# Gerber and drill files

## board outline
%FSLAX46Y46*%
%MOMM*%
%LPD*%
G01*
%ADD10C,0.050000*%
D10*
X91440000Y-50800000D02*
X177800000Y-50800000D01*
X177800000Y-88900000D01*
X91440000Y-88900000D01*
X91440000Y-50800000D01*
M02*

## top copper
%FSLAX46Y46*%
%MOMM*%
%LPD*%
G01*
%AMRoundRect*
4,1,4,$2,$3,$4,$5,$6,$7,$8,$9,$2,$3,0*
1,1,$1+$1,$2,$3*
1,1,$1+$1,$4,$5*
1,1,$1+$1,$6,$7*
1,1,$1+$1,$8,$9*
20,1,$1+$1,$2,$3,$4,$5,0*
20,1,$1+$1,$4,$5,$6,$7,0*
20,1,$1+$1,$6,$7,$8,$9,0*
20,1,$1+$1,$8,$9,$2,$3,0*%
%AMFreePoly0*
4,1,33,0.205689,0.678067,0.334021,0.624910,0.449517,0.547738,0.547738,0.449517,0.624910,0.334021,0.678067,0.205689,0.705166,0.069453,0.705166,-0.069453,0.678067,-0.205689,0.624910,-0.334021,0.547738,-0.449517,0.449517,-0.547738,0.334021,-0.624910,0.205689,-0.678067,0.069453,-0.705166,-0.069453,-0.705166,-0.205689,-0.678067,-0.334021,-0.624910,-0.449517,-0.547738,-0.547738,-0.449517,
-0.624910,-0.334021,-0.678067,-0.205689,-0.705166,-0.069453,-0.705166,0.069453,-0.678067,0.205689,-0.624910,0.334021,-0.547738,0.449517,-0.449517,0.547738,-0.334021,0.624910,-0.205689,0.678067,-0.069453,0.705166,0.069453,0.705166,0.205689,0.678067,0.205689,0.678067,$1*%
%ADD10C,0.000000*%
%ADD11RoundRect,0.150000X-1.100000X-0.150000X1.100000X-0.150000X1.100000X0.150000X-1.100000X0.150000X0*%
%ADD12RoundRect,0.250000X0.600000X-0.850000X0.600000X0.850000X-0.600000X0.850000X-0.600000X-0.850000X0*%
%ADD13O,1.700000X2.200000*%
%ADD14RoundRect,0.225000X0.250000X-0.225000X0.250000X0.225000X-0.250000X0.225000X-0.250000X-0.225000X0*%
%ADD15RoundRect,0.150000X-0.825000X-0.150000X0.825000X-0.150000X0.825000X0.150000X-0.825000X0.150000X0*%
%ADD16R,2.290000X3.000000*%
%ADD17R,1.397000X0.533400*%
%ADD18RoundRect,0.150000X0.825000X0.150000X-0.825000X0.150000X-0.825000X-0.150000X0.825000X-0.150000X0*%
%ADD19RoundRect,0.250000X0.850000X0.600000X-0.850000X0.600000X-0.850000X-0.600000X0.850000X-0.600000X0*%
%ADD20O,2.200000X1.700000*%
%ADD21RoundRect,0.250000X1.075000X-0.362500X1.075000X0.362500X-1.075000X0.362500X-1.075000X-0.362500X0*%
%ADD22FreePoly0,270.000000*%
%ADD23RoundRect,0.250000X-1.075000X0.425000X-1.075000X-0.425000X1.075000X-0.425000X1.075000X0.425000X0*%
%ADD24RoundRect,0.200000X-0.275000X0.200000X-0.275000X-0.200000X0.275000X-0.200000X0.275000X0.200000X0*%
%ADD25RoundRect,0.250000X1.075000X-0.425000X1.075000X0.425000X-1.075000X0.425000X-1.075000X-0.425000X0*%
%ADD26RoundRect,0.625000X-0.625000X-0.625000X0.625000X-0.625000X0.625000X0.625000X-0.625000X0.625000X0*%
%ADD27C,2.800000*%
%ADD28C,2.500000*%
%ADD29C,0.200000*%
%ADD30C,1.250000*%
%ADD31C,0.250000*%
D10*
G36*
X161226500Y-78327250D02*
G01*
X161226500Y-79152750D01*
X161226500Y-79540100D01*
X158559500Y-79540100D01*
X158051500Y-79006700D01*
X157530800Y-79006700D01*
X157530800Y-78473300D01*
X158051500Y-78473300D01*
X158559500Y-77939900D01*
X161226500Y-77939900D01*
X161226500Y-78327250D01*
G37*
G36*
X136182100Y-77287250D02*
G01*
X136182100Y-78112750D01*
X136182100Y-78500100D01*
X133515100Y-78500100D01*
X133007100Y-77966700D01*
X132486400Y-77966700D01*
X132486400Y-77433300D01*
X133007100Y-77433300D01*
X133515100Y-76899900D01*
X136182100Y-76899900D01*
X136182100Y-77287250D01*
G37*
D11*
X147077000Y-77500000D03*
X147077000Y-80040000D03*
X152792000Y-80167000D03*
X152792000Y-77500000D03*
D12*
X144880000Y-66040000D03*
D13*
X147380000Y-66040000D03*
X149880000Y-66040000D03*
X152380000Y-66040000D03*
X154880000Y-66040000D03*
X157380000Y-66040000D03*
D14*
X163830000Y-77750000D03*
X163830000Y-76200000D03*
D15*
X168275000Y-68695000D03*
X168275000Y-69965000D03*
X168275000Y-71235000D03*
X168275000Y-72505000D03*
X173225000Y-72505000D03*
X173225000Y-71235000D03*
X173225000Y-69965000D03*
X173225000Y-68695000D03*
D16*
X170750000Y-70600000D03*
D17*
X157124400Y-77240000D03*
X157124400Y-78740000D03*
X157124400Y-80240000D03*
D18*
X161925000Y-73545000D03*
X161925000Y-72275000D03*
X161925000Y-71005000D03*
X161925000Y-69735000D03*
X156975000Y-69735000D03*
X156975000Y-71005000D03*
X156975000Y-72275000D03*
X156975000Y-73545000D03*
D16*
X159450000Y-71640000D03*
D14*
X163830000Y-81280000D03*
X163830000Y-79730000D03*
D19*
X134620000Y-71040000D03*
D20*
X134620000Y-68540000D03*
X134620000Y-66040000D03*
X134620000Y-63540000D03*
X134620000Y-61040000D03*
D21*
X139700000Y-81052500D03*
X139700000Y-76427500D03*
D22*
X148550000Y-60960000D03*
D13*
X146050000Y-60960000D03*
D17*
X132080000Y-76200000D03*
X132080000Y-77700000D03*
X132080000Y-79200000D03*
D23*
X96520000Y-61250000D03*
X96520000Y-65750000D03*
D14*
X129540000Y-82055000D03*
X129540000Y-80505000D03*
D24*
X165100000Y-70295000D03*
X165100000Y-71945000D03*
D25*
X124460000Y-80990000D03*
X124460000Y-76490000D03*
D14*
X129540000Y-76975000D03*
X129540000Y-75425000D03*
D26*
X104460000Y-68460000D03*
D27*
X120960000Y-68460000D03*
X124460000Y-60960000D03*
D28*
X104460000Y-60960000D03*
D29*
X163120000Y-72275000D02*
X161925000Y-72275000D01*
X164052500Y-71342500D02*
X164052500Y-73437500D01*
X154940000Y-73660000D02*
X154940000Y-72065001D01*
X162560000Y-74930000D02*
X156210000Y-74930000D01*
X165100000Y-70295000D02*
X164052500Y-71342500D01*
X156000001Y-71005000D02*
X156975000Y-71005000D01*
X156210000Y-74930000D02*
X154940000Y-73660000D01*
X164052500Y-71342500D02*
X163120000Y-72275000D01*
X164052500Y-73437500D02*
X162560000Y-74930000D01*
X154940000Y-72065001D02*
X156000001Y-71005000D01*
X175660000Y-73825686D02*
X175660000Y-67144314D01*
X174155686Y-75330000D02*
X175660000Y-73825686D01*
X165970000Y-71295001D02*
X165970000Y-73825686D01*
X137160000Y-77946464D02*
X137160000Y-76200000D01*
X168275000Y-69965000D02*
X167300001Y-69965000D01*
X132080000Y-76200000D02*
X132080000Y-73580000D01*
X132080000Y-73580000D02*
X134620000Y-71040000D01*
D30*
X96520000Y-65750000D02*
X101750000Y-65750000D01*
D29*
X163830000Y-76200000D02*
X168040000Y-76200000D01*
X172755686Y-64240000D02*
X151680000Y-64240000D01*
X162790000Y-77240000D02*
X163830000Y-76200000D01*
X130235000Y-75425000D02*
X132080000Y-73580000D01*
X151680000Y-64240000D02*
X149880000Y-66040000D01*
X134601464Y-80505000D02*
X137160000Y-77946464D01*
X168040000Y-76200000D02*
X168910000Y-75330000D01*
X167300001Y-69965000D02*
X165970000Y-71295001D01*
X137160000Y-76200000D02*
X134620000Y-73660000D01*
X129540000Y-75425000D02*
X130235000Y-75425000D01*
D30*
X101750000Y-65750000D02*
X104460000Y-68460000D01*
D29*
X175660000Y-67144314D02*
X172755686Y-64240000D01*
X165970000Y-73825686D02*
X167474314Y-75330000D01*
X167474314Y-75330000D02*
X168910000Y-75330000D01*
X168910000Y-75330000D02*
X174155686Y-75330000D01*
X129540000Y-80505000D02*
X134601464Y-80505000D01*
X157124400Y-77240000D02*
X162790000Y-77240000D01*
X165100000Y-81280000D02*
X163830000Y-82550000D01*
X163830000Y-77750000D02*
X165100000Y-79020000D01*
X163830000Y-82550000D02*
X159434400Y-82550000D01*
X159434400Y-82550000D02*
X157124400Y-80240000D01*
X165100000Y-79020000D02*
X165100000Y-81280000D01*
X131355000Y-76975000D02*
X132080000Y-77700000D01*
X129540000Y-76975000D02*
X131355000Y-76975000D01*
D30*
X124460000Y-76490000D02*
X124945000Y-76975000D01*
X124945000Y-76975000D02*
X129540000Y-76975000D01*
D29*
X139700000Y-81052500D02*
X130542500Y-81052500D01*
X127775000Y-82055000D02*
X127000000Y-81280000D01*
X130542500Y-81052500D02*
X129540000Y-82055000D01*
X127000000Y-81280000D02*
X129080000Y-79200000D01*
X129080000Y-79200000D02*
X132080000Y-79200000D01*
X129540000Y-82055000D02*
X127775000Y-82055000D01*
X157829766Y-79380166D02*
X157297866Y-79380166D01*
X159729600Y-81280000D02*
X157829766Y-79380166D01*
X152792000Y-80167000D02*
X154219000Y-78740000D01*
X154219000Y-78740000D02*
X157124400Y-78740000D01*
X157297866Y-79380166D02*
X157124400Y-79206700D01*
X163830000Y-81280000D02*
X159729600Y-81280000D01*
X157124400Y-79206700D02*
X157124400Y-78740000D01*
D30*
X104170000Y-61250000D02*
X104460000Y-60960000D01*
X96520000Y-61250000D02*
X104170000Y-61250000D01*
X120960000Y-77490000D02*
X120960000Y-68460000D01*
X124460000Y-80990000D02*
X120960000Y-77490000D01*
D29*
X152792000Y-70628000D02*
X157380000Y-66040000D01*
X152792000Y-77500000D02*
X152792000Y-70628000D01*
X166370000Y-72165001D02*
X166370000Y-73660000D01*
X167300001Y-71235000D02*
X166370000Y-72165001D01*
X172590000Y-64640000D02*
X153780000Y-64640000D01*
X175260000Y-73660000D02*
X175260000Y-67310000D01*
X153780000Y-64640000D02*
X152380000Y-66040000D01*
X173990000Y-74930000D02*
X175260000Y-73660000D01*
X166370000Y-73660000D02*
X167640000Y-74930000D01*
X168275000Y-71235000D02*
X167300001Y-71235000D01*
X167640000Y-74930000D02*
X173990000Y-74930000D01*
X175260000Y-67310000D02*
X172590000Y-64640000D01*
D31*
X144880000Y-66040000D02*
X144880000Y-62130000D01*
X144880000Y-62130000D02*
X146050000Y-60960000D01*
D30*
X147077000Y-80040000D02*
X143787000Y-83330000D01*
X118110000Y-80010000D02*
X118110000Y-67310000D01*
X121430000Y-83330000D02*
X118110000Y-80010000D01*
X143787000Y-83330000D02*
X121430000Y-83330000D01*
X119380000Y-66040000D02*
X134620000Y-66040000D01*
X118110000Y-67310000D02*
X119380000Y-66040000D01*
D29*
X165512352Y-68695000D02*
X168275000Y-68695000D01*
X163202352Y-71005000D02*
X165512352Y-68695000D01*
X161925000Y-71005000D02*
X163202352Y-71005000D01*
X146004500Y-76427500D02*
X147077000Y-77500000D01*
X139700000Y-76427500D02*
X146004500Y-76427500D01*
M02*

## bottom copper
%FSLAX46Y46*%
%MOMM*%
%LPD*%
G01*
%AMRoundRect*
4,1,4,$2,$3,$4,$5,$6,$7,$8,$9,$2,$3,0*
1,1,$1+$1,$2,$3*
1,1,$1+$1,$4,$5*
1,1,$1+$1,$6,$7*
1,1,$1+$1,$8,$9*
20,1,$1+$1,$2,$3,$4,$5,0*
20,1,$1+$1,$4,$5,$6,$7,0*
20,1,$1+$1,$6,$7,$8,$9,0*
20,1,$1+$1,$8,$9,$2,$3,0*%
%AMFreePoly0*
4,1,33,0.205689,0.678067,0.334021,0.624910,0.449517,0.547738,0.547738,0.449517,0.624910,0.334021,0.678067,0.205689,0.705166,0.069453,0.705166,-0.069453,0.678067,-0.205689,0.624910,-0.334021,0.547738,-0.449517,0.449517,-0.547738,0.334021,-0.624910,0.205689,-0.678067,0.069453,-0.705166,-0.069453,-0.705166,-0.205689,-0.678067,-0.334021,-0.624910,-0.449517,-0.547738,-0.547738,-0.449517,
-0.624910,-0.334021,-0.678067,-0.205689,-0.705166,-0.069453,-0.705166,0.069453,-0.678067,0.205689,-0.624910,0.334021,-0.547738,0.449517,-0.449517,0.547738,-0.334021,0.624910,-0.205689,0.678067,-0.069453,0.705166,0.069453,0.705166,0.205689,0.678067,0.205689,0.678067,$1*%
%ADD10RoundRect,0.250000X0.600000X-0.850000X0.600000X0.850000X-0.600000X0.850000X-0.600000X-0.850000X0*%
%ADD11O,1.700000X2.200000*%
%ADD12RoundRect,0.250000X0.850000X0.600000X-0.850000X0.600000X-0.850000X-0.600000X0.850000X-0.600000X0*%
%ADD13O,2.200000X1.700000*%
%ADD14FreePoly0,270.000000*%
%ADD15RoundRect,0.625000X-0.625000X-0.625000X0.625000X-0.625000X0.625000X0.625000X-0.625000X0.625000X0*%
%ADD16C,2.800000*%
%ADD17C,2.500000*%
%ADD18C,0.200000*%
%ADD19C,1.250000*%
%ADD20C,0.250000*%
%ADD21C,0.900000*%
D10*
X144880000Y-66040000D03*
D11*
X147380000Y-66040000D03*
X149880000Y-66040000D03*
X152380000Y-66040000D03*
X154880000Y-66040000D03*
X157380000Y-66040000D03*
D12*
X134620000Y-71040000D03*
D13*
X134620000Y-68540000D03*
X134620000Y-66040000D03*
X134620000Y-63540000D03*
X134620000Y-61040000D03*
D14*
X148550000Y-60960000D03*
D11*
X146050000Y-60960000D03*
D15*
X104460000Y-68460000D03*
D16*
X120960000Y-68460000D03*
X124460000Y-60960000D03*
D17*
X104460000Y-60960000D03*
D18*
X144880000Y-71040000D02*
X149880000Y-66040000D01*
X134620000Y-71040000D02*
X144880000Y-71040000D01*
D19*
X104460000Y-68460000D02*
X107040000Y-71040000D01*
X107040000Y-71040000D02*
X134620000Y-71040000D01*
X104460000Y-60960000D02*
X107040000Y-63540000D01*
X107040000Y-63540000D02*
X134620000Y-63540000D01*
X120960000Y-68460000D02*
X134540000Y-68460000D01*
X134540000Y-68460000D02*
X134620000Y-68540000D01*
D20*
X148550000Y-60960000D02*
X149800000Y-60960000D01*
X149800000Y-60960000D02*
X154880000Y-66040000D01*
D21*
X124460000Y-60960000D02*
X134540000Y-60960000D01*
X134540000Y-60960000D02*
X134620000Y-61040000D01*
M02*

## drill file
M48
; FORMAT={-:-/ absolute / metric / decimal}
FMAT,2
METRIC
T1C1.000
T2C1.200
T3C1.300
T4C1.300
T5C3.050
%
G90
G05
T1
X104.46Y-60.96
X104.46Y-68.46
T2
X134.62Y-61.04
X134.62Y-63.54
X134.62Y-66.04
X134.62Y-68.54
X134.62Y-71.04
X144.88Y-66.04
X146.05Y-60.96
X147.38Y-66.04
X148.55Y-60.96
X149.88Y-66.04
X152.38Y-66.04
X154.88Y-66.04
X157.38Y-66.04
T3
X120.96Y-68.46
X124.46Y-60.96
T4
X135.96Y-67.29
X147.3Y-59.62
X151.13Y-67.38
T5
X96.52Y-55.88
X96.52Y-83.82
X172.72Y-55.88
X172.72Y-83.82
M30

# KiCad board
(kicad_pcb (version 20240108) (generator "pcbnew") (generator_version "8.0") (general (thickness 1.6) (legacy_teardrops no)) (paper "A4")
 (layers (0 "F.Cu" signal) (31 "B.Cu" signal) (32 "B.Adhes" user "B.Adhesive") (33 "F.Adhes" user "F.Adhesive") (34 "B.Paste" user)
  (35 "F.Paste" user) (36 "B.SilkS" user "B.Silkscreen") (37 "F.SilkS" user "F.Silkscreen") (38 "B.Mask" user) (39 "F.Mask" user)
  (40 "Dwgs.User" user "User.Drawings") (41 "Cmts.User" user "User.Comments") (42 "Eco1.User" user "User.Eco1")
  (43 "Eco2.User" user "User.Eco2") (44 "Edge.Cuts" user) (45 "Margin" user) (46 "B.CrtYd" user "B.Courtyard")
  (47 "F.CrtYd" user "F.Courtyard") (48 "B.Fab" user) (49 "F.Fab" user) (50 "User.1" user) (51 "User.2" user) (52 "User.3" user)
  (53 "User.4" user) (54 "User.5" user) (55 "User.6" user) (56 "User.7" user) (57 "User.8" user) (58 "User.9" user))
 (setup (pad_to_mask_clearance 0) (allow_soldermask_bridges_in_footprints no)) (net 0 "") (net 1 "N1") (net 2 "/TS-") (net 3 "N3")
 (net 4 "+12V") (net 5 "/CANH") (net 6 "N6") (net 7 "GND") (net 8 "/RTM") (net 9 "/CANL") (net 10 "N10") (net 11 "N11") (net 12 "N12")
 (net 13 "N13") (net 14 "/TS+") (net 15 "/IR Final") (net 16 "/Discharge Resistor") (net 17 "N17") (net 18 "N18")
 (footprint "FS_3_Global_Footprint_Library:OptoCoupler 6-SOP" (layer "F.Cu") (at 149.86 78.74)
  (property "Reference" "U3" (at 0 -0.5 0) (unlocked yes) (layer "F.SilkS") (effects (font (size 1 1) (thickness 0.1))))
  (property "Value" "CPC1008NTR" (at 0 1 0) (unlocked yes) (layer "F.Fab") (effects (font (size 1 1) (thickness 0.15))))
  (pad "1" smd roundrect (at -2.783 -1.24) (size 2.5 0.6) (layers "F.Cu" "F.Paste" "F.Mask") (roundrect_rratio 0.25) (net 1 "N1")
   (thermal_bridge_angle 45))
  (pad "3" smd roundrect (at -2.783 1.3) (size 2.5 0.6) (layers "F.Cu" "F.Paste" "F.Mask") (roundrect_rratio 0.25) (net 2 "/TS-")
   (thermal_bridge_angle 45))
  (pad "4" smd roundrect (at 2.932 1.427) (size 2.5 0.6) (layers "F.Cu" "F.Paste" "F.Mask") (roundrect_rratio 0.25) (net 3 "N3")
   (thermal_bridge_angle 45))
  (pad "6" smd roundrect (at 2.932 -1.24) (size 2.5 0.6) (layers "F.Cu" "F.Paste" "F.Mask") (roundrect_rratio 0.25) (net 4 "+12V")
   (thermal_bridge_angle 45)))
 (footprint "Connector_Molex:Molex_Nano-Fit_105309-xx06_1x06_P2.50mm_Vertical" (layer "F.Cu") (at 144.88 66.04 90)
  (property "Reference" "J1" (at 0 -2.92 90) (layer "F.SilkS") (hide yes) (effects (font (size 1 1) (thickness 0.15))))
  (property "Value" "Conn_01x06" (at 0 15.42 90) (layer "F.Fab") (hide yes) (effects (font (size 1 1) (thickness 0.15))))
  (pad "" np_thru_hole circle (at -1.34 6.25 90) (size 1.3 1.3) (drill 1.3) (layers "*.Cu" "*.Mask"))
  (pad "1" thru_hole roundrect (at 0 0 90) (size 2.2 1.7) (drill 1.2) (layers "*.Cu" "*.Mask") (remove_unused_layers no)
   (roundrect_rratio 0.147059) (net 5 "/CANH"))
  (pad "2" thru_hole oval (at 0 2.5 90) (size 2.2 1.7) (drill 1.2) (layers "*.Cu" "*.Mask") (remove_unused_layers no) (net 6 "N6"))
  (pad "3" thru_hole oval (at 0 5 90) (size 2.2 1.7) (drill 1.2) (layers "*.Cu" "*.Mask") (remove_unused_layers no) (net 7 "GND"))
  (pad "4" thru_hole oval (at 0 7.5 90) (size 2.2 1.7) (drill 1.2) (layers "*.Cu" "*.Mask") (remove_unused_layers no) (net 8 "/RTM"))
  (pad "5" thru_hole oval (at 0 10 90) (size 2.2 1.7) (drill 1.2) (layers "*.Cu" "*.Mask") (remove_unused_layers no) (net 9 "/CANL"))
  (pad "6" thru_hole oval (at 0 12.5 90) (size 2.2 1.7) (drill 1.2) (layers "*.Cu" "*.Mask") (remove_unused_layers no) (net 4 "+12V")))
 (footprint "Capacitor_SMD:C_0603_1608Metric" (layer "F.Cu") (at 163.83 76.975 90)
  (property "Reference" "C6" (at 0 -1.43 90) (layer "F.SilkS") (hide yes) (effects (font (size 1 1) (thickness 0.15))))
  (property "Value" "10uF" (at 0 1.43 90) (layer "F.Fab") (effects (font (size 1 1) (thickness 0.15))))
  (pad "1" smd roundrect (at -0.775 0 90) (size 0.9 0.95) (layers "F.Cu" "F.Paste" "F.Mask") (roundrect_rratio 0.25) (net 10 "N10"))
  (pad "2" smd roundrect (at 0.775 0 90) (size 0.9 0.95) (layers "F.Cu" "F.Paste" "F.Mask") (roundrect_rratio 0.25) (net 7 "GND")))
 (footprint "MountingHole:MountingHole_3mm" (layer "F.Cu") (at 96.52 55.88)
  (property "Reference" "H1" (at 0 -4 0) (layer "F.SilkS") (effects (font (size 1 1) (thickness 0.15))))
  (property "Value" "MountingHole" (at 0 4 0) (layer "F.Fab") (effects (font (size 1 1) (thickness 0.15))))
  (pad "" np_thru_hole circle (at 0 0) (size 3.05 3.05) (drill 3.05) (layers "F&B.Cu" "*.Mask")))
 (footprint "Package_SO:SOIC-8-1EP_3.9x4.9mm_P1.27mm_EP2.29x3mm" (layer "F.Cu") (at 170.75 70.6)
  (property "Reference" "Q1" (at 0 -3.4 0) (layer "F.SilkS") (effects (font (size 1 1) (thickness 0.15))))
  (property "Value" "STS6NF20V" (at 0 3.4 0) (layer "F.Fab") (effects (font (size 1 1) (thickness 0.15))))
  (pad "" smd roundrect (at -0.57 -0.75) (size 0.92 1.21) (layers "F.Paste") (roundrect_rratio 0.25))
  (pad "" smd roundrect (at -0.57 0.75) (size 0.92 1.21) (layers "F.Paste") (roundrect_rratio 0.25))
  (pad "" smd roundrect (at 0.57 -0.75) (size 0.92 1.21) (layers "F.Paste") (roundrect_rratio 0.25))
  (pad "" smd roundrect (at 0.57 0.75) (size 0.92 1.21) (layers "F.Paste") (roundrect_rratio 0.25))
  (pad "1" smd roundrect (at -2.475 -1.905) (size 1.95 0.6) (layers "F.Cu" "F.Paste" "F.Mask") (roundrect_rratio 0.25) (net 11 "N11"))
  (pad "2" smd roundrect (at -2.475 -0.635) (size 1.95 0.6) (layers "F.Cu" "F.Paste" "F.Mask") (roundrect_rratio 0.25) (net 7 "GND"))
  (pad "3" smd roundrect (at -2.475 0.635) (size 1.95 0.6) (layers "F.Cu" "F.Paste" "F.Mask") (roundrect_rratio 0.25) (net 8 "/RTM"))
  (pad "4" smd roundrect (at -2.475 1.905) (size 1.95 0.6) (layers "F.Cu" "F.Paste" "F.Mask") (roundrect_rratio 0.25))
  (pad "5" smd roundrect (at 2.475 1.905) (size 1.95 0.6) (layers "F.Cu" "F.Paste" "F.Mask") (roundrect_rratio 0.25))
  (pad "6" smd roundrect (at 2.475 0.635) (size 1.95 0.6) (layers "F.Cu" "F.Paste" "F.Mask") (roundrect_rratio 0.25))
  (pad "7" smd roundrect (at 2.475 -0.635) (size 1.95 0.6) (layers "F.Cu" "F.Paste" "F.Mask") (roundrect_rratio 0.25))
  (pad "8" smd roundrect (at 2.475 -1.905) (size 1.95 0.6) (layers "F.Cu" "F.Paste" "F.Mask") (roundrect_rratio 0.25))
  (pad "9" smd rect (at 0 0) (size 2.29 3) (layers "F.Cu" "F.Mask") (zone_connect 2)))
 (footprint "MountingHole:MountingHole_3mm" (layer "F.Cu") (at 172.72 83.82)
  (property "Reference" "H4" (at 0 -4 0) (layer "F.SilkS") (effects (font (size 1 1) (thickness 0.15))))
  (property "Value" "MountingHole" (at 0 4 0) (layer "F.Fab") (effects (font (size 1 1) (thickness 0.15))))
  (pad "" np_thru_hole circle (at 0 0) (size 3.05 3.05) (drill 3.05) (layers "F&B.Cu" "*.Mask")))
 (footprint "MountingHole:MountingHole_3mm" (layer "F.Cu") (at 172.72 55.88)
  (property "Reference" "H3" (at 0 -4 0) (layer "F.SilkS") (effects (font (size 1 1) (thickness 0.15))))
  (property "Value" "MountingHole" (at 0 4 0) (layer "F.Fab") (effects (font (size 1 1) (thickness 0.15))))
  (pad "" np_thru_hole circle (at 0 0) (size 3.05 3.05) (drill 3.05) (layers "F&B.Cu" "*.Mask")))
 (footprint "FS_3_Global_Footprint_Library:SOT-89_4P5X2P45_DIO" (layer "F.Cu") (at 158.75 78.74 -90)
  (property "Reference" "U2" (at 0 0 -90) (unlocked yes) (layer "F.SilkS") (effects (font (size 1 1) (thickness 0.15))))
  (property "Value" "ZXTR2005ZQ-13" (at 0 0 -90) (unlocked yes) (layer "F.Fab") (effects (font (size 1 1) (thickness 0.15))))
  (fp_poly
   (pts (xy -0.2667 1.2192) (xy -0.2667 0.6985) (xy -0.8001 0.1905) (xy -0.8001 -2.4765) (xy -0.41275 -2.4765) (xy 0.41275 -2.4765)
    (xy 0.8001 -2.4765) (xy 0.8001 0.1905) (xy 0.2667 0.6985) (xy 0.2667 1.2192))
   (stroke (width 0) (type solid)) (fill solid) (layer "F.Cu"))
  (pad "1" smd rect (at -1.5 1.6256 270) (size 0.5334 1.397) (layers "F.Cu" "F.Paste" "F.Mask") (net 7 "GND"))
  (pad "2" smd rect (at 0 1.6256 270) (size 0.5334 1.397) (layers "F.Cu" "F.Paste" "F.Mask") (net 3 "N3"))
  (pad "3" smd rect (at 1.5 1.6256 270) (size 0.5334 1.397) (layers "F.Cu" "F.Paste" "F.Mask") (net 10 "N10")))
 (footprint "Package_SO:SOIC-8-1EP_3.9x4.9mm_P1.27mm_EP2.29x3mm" (layer "F.Cu") (at 159.45 71.64 180)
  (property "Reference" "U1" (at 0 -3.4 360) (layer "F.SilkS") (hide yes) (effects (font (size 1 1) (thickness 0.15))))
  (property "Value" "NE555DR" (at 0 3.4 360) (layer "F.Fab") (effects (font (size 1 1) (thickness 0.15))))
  (pad "" smd roundrect (at -0.57 -0.75 180) (size 0.92 1.21) (layers "F.Paste") (roundrect_rratio 0.25))
  (pad "" smd roundrect (at -0.57 0.75 180) (size 0.92 1.21) (layers "F.Paste") (roundrect_rratio 0.25))
  (pad "" smd roundrect (at 0.57 -0.75 180) (size 0.92 1.21) (layers "F.Paste") (roundrect_rratio 0.25))
  (pad "" smd roundrect (at 0.57 0.75 180) (size 0.92 1.21) (layers "F.Paste") (roundrect_rratio 0.25))
  (pad "1" smd roundrect (at -2.475 -1.905 180) (size 1.95 0.6) (layers "F.Cu" "F.Paste" "F.Mask") (roundrect_rratio 0.25) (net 7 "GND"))
  (pad "2" smd roundrect (at -2.475 -0.635 180) (size 1.95 0.6) (layers "F.Cu" "F.Paste" "F.Mask") (roundrect_rratio 0.25) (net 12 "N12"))
  (pad "3" smd roundrect (at -2.475 0.635 180) (size 1.95 0.6) (layers "F.Cu" "F.Paste" "F.Mask") (roundrect_rratio 0.25) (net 11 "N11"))
  (pad "4" smd roundrect (at -2.475 1.905 180) (size 1.95 0.6) (layers "F.Cu" "F.Paste" "F.Mask") (roundrect_rratio 0.25) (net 10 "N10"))
  (pad "5" smd roundrect (at 2.475 1.905 180) (size 1.95 0.6) (layers "F.Cu" "F.Paste" "F.Mask") (roundrect_rratio 0.25) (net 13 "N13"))
  (pad "6" smd roundrect (at 2.475 0.635 180) (size 1.95 0.6) (layers "F.Cu" "F.Paste" "F.Mask") (roundrect_rratio 0.25) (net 12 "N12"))
  (pad "7" smd roundrect (at 2.475 -0.635 180) (size 1.95 0.6) (layers "F.Cu" "F.Paste" "F.Mask") (roundrect_rratio 0.25) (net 10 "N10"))
  (pad "8" smd roundrect (at 2.475 -1.905 180) (size 1.95 0.6) (layers "F.Cu" "F.Paste" "F.Mask") (roundrect_rratio 0.25) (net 10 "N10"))
  (pad "9" smd rect (at 0 0 180) (size 2.29 3) (layers "F.Cu" "F.Mask") (zone_connect 2)))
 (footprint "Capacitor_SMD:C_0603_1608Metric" (layer "F.Cu") (at 163.83 80.505 90)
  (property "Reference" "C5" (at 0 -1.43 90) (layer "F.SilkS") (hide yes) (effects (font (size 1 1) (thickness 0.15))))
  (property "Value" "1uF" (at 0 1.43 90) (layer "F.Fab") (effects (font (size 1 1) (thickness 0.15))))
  (pad "1" smd roundrect (at -0.775 0 90) (size 0.9 0.95) (layers "F.Cu" "F.Paste" "F.Mask") (roundrect_rratio 0.25) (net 3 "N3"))
  (pad "2" smd roundrect (at 0.775 0 90) (size 0.9 0.95) (layers "F.Cu" "F.Paste" "F.Mask") (roundrect_rratio 0.25) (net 7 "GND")))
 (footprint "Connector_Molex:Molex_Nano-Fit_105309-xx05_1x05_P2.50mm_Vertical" (layer "F.Cu") (at 134.62 71.04 180)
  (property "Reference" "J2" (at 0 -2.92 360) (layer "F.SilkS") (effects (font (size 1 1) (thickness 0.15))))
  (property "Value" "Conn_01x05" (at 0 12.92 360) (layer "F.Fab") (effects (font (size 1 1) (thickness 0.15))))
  (pad "" np_thru_hole circle (at -1.34 3.75 180) (size 1.3 1.3) (drill 1.3) (layers "*.Cu" "*.Mask"))
  (pad "1" thru_hole roundrect (at 0 0 180) (size 2.2 1.7) (drill 1.2) (layers "*.Cu" "*.Mask") (remove_unused_layers no)
   (roundrect_rratio 0.147059) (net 7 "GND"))
  (pad "2" thru_hole oval (at 0 2.5 180) (size 2.2 1.7) (drill 1.2) (layers "*.Cu" "*.Mask") (remove_unused_layers no) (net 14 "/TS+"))
  (pad "3" thru_hole oval (at 0 5 180) (size 2.2 1.7) (drill 1.2) (layers "*.Cu" "*.Mask") (remove_unused_layers no) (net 2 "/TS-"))
  (pad "4" thru_hole oval (at 0 7.5 180) (size 2.2 1.7) (drill 1.2) (layers "*.Cu" "*.Mask") (remove_unused_layers no) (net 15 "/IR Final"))
  (pad "5" thru_hole oval (at 0 10 180) (size 2.2 1.7) (drill 1.2) (layers "*.Cu" "*.Mask") (remove_unused_layers no)
   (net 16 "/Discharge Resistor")))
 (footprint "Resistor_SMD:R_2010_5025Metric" (layer "F.Cu") (at 139.7 78.74 90)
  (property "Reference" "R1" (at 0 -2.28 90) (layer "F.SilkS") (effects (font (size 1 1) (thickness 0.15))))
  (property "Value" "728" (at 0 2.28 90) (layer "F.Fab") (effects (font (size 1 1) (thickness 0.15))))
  (pad "1" smd roundrect (at -2.3125 0 90) (size 1.225 2.65) (layers "F.Cu" "F.Paste" "F.Mask") (roundrect_rratio 0.204082) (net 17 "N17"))
  (pad "2" smd roundrect (at 2.3125 0 90) (size 1.225 2.65) (layers "F.Cu" "F.Paste" "F.Mask") (roundrect_rratio 0.204082) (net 1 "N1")))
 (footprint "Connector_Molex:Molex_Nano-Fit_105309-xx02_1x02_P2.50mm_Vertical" (layer "F.Cu") (at 148.55 60.96 -90)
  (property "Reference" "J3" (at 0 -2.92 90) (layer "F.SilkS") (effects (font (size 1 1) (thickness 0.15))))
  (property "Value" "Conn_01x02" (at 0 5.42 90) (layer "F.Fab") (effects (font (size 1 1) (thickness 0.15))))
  (pad "" np_thru_hole circle (at -1.34 1.25 270) (size 1.3 1.3) (drill 1.3) (layers "*.Cu" "*.Mask"))
  (pad "1" thru_hole custom (at 0 0 270) (size 1.417157 1.417157) (drill 1.2) (layers "*.Cu" "*.Mask") (remove_unused_layers no)
   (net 9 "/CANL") (thermal_bridge_angle 90) (options (clearance outline) (anchor circle)) (primitives))
  (pad "2" thru_hole oval (at 0 2.5 270) (size 2.2 1.7) (drill 1.2) (layers "*.Cu" "*.Mask") (remove_unused_layers no) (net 5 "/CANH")))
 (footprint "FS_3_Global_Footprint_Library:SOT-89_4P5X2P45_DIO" (layer "F.Cu") (at 133.7056 77.7 -90)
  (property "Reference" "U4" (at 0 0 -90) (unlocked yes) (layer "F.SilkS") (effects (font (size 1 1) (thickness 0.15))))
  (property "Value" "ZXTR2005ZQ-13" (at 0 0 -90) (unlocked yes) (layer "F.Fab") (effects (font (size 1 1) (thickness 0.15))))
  (fp_poly
   (pts (xy -0.2667 1.2192) (xy -0.2667 0.6985) (xy -0.8001 0.1905) (xy -0.8001 -2.4765) (xy -0.41275 -2.4765) (xy 0.41275 -2.4765)
    (xy 0.8001 -2.4765) (xy 0.8001 0.1905) (xy 0.2667 0.6985) (xy 0.2667 1.2192))
   (stroke (width 0) (type solid)) (fill solid) (layer "F.Cu"))
  (pad "1" smd rect (at -1.5 1.6256 270) (size 0.5334 1.397) (layers "F.Cu" "F.Paste" "F.Mask") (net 7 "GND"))
  (pad "2" smd rect (at 0 1.6256 270) (size 0.5334 1.397) (layers "F.Cu" "F.Paste" "F.Mask") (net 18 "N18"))
  (pad "3" smd rect (at 1.5 1.6256 270) (size 0.5334 1.397) (layers "F.Cu" "F.Paste" "F.Mask") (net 17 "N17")))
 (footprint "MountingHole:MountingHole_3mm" (layer "F.Cu") (at 96.52 83.82)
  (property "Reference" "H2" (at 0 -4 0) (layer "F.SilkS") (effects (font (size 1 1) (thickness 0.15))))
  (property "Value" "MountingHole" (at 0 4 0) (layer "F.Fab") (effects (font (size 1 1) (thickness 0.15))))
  (pad "" np_thru_hole circle (at 0 0) (size 3.05 3.05) (drill 3.05) (layers "F&B.Cu" "*.Mask")))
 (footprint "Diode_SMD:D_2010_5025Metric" (layer "F.Cu") (at 96.52 63.5 -90)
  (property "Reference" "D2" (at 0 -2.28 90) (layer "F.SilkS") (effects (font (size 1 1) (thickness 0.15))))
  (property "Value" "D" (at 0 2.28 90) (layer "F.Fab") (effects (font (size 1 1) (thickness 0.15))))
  (pad "1" smd roundrect (at -2.25 0 270) (size 1.35 2.65) (layers "F.Cu" "F.Paste" "F.Mask") (roundrect_rratio 0.185185)
   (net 15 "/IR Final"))
  (pad "2" smd roundrect (at 2.25 0 270) (size 1.35 2.65) (layers "F.Cu" "F.Paste" "F.Mask") (roundrect_rratio 0.185185) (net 7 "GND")))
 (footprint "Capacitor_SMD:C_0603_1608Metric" (layer "F.Cu") (at 129.54 81.28 90)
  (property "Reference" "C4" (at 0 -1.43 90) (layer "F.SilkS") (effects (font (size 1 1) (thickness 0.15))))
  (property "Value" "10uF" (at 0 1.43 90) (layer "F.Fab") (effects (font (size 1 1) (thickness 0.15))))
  (pad "1" smd roundrect (at -0.775 0 90) (size 0.9 0.95) (layers "F.Cu" "F.Paste" "F.Mask") (roundrect_rratio 0.25) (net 17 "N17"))
  (pad "2" smd roundrect (at 0.775 0 90) (size 0.9 0.95) (layers "F.Cu" "F.Paste" "F.Mask") (roundrect_rratio 0.25) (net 7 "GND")))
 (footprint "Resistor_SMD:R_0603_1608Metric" (layer "F.Cu") (at 165.1 71.12 -90)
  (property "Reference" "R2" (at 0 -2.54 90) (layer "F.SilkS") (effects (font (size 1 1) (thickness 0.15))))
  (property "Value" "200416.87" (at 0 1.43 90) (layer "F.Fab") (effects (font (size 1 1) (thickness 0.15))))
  (pad "1" smd roundrect (at -0.825 0 270) (size 0.8 0.95) (layers "F.Cu" "F.Paste" "F.Mask") (roundrect_rratio 0.25) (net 12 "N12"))
  (pad "2" smd roundrect (at 0.825 0 270) (size 0.8 0.95) (layers "F.Cu" "F.Paste" "F.Mask") (roundrect_rratio 0.25) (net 10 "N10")))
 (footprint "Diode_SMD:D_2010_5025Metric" (layer "F.Cu") (at 124.46 78.74 90)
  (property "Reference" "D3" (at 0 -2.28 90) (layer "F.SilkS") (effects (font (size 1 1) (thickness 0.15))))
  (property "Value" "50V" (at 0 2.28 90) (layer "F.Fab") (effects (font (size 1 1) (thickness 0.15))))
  (pad "1" smd roundrect (at -2.25 0 90) (size 1.35 2.65) (layers "F.Cu" "F.Paste" "F.Mask") (roundrect_rratio 0.185185) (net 14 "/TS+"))
  (pad "2" smd roundrect (at 2.25 0 90) (size 1.35 2.65) (layers "F.Cu" "F.Paste" "F.Mask") (roundrect_rratio 0.185185) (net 18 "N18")))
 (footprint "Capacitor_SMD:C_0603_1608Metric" (layer "F.Cu") (at 129.54 76.2 90)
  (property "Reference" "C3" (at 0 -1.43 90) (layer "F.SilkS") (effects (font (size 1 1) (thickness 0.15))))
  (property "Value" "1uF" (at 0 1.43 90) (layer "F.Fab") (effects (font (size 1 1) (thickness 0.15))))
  (pad "1" smd roundrect (at -0.775 0 90) (size 0.9 0.95) (layers "F.Cu" "F.Paste" "F.Mask") (roundrect_rratio 0.25) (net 18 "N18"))
  (pad "2" smd roundrect (at 0.775 0 90) (size 0.9 0.95) (layers "F.Cu" "F.Paste" "F.Mask") (roundrect_rratio 0.25) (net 7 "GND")))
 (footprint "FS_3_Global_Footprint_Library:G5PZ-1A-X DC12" (layer "F.Cu") (at 101.92 57.12)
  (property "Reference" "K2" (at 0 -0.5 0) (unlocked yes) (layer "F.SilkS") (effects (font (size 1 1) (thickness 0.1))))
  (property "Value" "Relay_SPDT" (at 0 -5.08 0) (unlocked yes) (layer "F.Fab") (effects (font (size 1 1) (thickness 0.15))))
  (pad "1" thru_hole roundrect (at 2.54 11.34) (size 2.5 2.5) (drill 1) (layers "*.Cu" "*.Mask") (remove_unused_layers no)
   (roundrect_rratio 0.25) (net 7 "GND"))
  (pad "2" thru_hole circle (at 19.04 11.34) (size 2.8 2.8) (drill 1.3) (layers "*.Cu" "*.Mask") (remove_unused_layers no) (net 14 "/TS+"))
  (pad "3" thru_hole circle (at 22.54 3.84) (size 2.8 2.8) (drill 1.3) (layers "*.Cu" "*.Mask") (remove_unused_layers no)
   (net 16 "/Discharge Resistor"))
  (pad "4" thru_hole circle (at 2.54 3.84) (size 2.5 2.5) (drill 1) (layers "*.Cu" "*.Mask") (remove_unused_layers no) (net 15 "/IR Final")))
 (gr_rect (start 91.44 50.8) (end 177.8 88.9) (stroke (width 0.05) (type default)) (fill none) (layer "Edge.Cuts"))
 (segment (start 163.12 72.275) (end 161.925 72.275) (width 0.2) (layer "F.Cu") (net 12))
 (segment (start 164.0525 71.3425) (end 164.0525 73.4375) (width 0.2) (layer "F.Cu") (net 12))
 (segment (start 154.94 73.66) (end 154.94 72.065001) (width 0.2) (layer "F.Cu") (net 12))
 (segment (start 162.56 74.93) (end 156.21 74.93) (width 0.2) (layer "F.Cu") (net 12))
 (segment (start 165.1 70.295) (end 164.0525 71.3425) (width 0.2) (layer "F.Cu") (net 12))
 (segment (start 156.000001 71.005) (end 156.975 71.005) (width 0.2) (layer "F.Cu") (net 12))
 (segment (start 156.21 74.93) (end 154.94 73.66) (width 0.2) (layer "F.Cu") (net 12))
 (segment (start 164.0525 71.3425) (end 163.12 72.275) (width 0.2) (layer "F.Cu") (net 12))
 (segment (start 164.0525 73.4375) (end 162.56 74.93) (width 0.2) (layer "F.Cu") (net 12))
 (segment (start 154.94 72.065001) (end 156.000001 71.005) (width 0.2) (layer "F.Cu") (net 12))
 (segment (start 175.66 73.825686) (end 175.66 67.144314) (width 0.2) (layer "F.Cu") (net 7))
 (segment (start 174.155686 75.33) (end 175.66 73.825686) (width 0.2) (layer "F.Cu") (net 7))
 (segment (start 165.97 71.295001) (end 165.97 73.825686) (width 0.2) (layer "F.Cu") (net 7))
 (segment (start 137.16 77.946464) (end 137.16 76.2) (width 0.2) (layer "F.Cu") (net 7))
 (segment (start 168.275 69.965) (end 167.300001 69.965) (width 0.2) (layer "F.Cu") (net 7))
 (segment (start 132.08 76.2) (end 132.08 73.58) (width 0.2) (layer "F.Cu") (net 7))
 (segment (start 132.08 73.58) (end 134.62 71.04) (width 0.2) (layer "F.Cu") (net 7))
 (segment (start 96.52 65.75) (end 101.75 65.75) (width 1.25) (layer "F.Cu") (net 7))
 (segment (start 163.83 76.2) (end 168.04 76.2) (width 0.2) (layer "F.Cu") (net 7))
 (segment (start 172.755686 64.24) (end 151.68 64.24) (width 0.2) (layer "F.Cu") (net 7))
 (segment (start 162.79 77.24) (end 163.83 76.2) (width 0.2) (layer "F.Cu") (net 7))
 (segment (start 130.235 75.425) (end 132.08 73.58) (width 0.2) (layer "F.Cu") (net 7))
 (segment (start 151.68 64.24) (end 149.88 66.04) (width 0.2) (layer "F.Cu") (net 7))
 (segment (start 134.601464 80.505) (end 137.16 77.946464) (width 0.2) (layer "F.Cu") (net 7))
 (segment (start 168.04 76.2) (end 168.91 75.33) (width 0.2) (layer "F.Cu") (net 7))
 (segment (start 167.300001 69.965) (end 165.97 71.295001) (width 0.2) (layer "F.Cu") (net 7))
 (segment (start 137.16 76.2) (end 134.62 73.66) (width 0.2) (layer "F.Cu") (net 7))
 (segment (start 129.54 75.425) (end 130.235 75.425) (width 0.2) (layer "F.Cu") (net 7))
 (segment (start 101.75 65.75) (end 104.46 68.46) (width 1.25) (layer "F.Cu") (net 7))
 (segment (start 175.66 67.144314) (end 172.755686 64.24) (width 0.2) (layer "F.Cu") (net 7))
 (segment (start 165.97 73.825686) (end 167.474314 75.33) (width 0.2) (layer "F.Cu") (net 7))
 (segment (start 167.474314 75.33) (end 168.91 75.33) (width 0.2) (layer "F.Cu") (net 7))
 (segment (start 168.91 75.33) (end 174.155686 75.33) (width 0.2) (layer "F.Cu") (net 7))
 (segment (start 129.54 80.505) (end 134.601464 80.505) (width 0.2) (layer "F.Cu") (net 7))
 (segment (start 157.1244 77.24) (end 162.79 77.24) (width 0.2) (layer "F.Cu") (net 7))
 (segment (start 144.88 71.04) (end 149.88 66.04) (width 0.2) (layer "B.Cu") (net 7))
 (segment (start 134.62 71.04) (end 144.88 71.04) (width 0.2) (layer "B.Cu") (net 7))
 (segment (start 104.46 68.46) (end 107.04 71.04) (width 1.25) (layer "B.Cu") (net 7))
 (segment (start 107.04 71.04) (end 134.62 71.04) (width 1.25) (layer "B.Cu") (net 7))
 (segment (start 165.1 81.28) (end 163.83 82.55) (width 0.2) (layer "F.Cu") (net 10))
 (segment (start 163.83 77.75) (end 165.1 79.02) (width 0.2) (layer "F.Cu") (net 10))
 (segment (start 163.83 82.55) (end 159.4344 82.55) (width 0.2) (layer "F.Cu") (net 10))
 (segment (start 159.4344 82.55) (end 157.1244 80.24) (width 0.2) (layer "F.Cu") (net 10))
 (segment (start 165.1 79.02) (end 165.1 81.28) (width 0.2) (layer "F.Cu") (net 10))
 (segment (start 131.355 76.975) (end 132.08 77.7) (width 0.2) (layer "F.Cu") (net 18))
 (segment (start 129.54 76.975) (end 131.355 76.975) (width 0.2) (layer "F.Cu") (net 18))
 (segment (start 124.46 76.49) (end 124.945 76.975) (width 1.25) (layer "F.Cu") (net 18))
 (segment (start 124.945 76.975) (end 129.54 76.975) (width 1.25) (layer "F.Cu") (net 18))
 (segment (start 139.7 81.0525) (end 130.5425 81.0525) (width 0.2) (layer "F.Cu") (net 17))
 (segment (start 127.775 82.055) (end 127 81.28) (width 0.2) (layer "F.Cu") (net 17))
 (segment (start 130.5425 81.0525) (end 129.54 82.055) (width 0.2) (layer "F.Cu") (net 17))
 (segment (start 127 81.28) (end 129.08 79.2) (width 0.2) (layer "F.Cu") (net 17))
 (segment (start 129.08 79.2) (end 132.08 79.2) (width 0.2) (layer "F.Cu") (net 17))
 (segment (start 129.54 82.055) (end 127.775 82.055) (width 0.2) (layer "F.Cu") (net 17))
 (segment (start 157.829766 79.380166) (end 157.297866 79.380166) (width 0.2) (layer "F.Cu") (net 3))
 (segment (start 159.7296 81.28) (end 157.829766 79.380166) (width 0.2) (layer "F.Cu") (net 3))
 (segment (start 152.792 80.167) (end 154.219 78.74) (width 0.2) (layer "F.Cu") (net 3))
 (segment (start 154.219 78.74) (end 157.1244 78.74) (width 0.2) (layer "F.Cu") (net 3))
 (segment (start 157.297866 79.380166) (end 157.1244 79.2067) (width 0.2) (layer "F.Cu") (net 3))
 (segment (start 163.83 81.28) (end 159.7296 81.28) (width 0.2) (layer "F.Cu") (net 3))
 (segment (start 157.1244 79.2067) (end 157.1244 78.74) (width 0.2) (layer "F.Cu") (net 3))
 (segment (start 104.17 61.25) (end 104.46 60.96) (width 1.25) (layer "F.Cu") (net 15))
 (segment (start 96.52 61.25) (end 104.17 61.25) (width 1.25) (layer "F.Cu") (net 15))
 (segment (start 104.46 60.96) (end 107.04 63.54) (width 1.25) (layer "B.Cu") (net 15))
 (segment (start 107.04 63.54) (end 134.62 63.54) (width 1.25) (layer "B.Cu") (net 15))
 (segment (start 120.96 77.49) (end 120.96 68.46) (width 1.25) (layer "F.Cu") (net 14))
 (segment (start 124.46 80.99) (end 120.96 77.49) (width 1.25) (layer "F.Cu") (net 14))
 (segment (start 120.96 68.46) (end 134.54 68.46) (width 1.25) (layer "B.Cu") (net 14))
 (segment (start 134.54 68.46) (end 134.62 68.54) (width 1.25) (layer "B.Cu") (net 14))
 (segment (start 152.792 70.628) (end 157.38 66.04) (width 0.2) (layer "F.Cu") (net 4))
 (segment (start 152.792 77.5) (end 152.792 70.628) (width 0.2) (layer "F.Cu") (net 4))
 (segment (start 166.37 72.165001) (end 166.37 73.66) (width 0.2) (layer "F.Cu") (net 8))
 (segment (start 167.300001 71.235) (end 166.37 72.165001) (width 0.2) (layer "F.Cu") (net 8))
 (segment (start 172.59 64.64) (end 153.78 64.64) (width 0.2) (layer "F.Cu") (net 8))
 (segment (start 175.26 73.66) (end 175.26 67.31) (width 0.2) (layer "F.Cu") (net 8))
 (segment (start 153.78 64.64) (end 152.38 66.04) (width 0.2) (layer "F.Cu") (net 8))
 (segment (start 173.99 74.93) (end 175.26 73.66) (width 0.2) (layer "F.Cu") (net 8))
 (segment (start 166.37 73.66) (end 167.64 74.93) (width 0.2) (layer "F.Cu") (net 8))
 (segment (start 168.275 71.235) (end 167.300001 71.235) (width 0.2) (layer "F.Cu") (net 8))
 (segment (start 167.64 74.93) (end 173.99 74.93) (width 0.2) (layer "F.Cu") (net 8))
 (segment (start 175.26 67.31) (end 172.59 64.64) (width 0.2) (layer "F.Cu") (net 8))
 (segment (start 148.55 60.96) (end 149.8 60.96) (width 0.25) (layer "B.Cu") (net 9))
 (segment (start 149.8 60.96) (end 154.88 66.04) (width 0.25) (layer "B.Cu") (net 9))
 (segment (start 144.88 66.04) (end 144.88 62.13) (width 0.25) (layer "F.Cu") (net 5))
 (segment (start 144.88 62.13) (end 146.05 60.96) (width 0.25) (layer "F.Cu") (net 5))
 (segment (start 124.46 60.96) (end 134.54 60.96) (width 0.9) (layer "B.Cu") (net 16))
 (segment (start 134.54 60.96) (end 134.62 61.04) (width 0.9) (layer "B.Cu") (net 16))
 (segment (start 147.077 80.04) (end 143.787 83.33) (width 1.25) (layer "F.Cu") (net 2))
 (segment (start 118.11 80.01) (end 118.11 67.31) (width 1.25) (layer "F.Cu") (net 2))
 (segment (start 121.43 83.33) (end 118.11 80.01) (width 1.25) (layer "F.Cu") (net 2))
 (segment (start 143.787 83.33) (end 121.43 83.33) (width 1.25) (layer "F.Cu") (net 2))
 (segment (start 119.38 66.04) (end 134.62 66.04) (width 1.25) (layer "F.Cu") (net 2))
 (segment (start 118.11 67.31) (end 119.38 66.04) (width 1.25) (layer "F.Cu") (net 2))
 (segment (start 165.512352 68.695) (end 168.275 68.695) (width 0.2) (layer "F.Cu") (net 11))
 (segment (start 163.202352 71.005) (end 165.512352 68.695) (width 0.2) (layer "F.Cu") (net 11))
 (segment (start 161.925 71.005) (end 163.202352 71.005) (width 0.2) (layer "F.Cu") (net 11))
 (segment (start 146.0045 76.4275) (end 147.077 77.5) (width 0.2) (layer "F.Cu") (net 1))
 (segment (start 139.7 76.4275) (end 146.0045 76.4275) (width 0.2) (layer "F.Cu") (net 1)))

